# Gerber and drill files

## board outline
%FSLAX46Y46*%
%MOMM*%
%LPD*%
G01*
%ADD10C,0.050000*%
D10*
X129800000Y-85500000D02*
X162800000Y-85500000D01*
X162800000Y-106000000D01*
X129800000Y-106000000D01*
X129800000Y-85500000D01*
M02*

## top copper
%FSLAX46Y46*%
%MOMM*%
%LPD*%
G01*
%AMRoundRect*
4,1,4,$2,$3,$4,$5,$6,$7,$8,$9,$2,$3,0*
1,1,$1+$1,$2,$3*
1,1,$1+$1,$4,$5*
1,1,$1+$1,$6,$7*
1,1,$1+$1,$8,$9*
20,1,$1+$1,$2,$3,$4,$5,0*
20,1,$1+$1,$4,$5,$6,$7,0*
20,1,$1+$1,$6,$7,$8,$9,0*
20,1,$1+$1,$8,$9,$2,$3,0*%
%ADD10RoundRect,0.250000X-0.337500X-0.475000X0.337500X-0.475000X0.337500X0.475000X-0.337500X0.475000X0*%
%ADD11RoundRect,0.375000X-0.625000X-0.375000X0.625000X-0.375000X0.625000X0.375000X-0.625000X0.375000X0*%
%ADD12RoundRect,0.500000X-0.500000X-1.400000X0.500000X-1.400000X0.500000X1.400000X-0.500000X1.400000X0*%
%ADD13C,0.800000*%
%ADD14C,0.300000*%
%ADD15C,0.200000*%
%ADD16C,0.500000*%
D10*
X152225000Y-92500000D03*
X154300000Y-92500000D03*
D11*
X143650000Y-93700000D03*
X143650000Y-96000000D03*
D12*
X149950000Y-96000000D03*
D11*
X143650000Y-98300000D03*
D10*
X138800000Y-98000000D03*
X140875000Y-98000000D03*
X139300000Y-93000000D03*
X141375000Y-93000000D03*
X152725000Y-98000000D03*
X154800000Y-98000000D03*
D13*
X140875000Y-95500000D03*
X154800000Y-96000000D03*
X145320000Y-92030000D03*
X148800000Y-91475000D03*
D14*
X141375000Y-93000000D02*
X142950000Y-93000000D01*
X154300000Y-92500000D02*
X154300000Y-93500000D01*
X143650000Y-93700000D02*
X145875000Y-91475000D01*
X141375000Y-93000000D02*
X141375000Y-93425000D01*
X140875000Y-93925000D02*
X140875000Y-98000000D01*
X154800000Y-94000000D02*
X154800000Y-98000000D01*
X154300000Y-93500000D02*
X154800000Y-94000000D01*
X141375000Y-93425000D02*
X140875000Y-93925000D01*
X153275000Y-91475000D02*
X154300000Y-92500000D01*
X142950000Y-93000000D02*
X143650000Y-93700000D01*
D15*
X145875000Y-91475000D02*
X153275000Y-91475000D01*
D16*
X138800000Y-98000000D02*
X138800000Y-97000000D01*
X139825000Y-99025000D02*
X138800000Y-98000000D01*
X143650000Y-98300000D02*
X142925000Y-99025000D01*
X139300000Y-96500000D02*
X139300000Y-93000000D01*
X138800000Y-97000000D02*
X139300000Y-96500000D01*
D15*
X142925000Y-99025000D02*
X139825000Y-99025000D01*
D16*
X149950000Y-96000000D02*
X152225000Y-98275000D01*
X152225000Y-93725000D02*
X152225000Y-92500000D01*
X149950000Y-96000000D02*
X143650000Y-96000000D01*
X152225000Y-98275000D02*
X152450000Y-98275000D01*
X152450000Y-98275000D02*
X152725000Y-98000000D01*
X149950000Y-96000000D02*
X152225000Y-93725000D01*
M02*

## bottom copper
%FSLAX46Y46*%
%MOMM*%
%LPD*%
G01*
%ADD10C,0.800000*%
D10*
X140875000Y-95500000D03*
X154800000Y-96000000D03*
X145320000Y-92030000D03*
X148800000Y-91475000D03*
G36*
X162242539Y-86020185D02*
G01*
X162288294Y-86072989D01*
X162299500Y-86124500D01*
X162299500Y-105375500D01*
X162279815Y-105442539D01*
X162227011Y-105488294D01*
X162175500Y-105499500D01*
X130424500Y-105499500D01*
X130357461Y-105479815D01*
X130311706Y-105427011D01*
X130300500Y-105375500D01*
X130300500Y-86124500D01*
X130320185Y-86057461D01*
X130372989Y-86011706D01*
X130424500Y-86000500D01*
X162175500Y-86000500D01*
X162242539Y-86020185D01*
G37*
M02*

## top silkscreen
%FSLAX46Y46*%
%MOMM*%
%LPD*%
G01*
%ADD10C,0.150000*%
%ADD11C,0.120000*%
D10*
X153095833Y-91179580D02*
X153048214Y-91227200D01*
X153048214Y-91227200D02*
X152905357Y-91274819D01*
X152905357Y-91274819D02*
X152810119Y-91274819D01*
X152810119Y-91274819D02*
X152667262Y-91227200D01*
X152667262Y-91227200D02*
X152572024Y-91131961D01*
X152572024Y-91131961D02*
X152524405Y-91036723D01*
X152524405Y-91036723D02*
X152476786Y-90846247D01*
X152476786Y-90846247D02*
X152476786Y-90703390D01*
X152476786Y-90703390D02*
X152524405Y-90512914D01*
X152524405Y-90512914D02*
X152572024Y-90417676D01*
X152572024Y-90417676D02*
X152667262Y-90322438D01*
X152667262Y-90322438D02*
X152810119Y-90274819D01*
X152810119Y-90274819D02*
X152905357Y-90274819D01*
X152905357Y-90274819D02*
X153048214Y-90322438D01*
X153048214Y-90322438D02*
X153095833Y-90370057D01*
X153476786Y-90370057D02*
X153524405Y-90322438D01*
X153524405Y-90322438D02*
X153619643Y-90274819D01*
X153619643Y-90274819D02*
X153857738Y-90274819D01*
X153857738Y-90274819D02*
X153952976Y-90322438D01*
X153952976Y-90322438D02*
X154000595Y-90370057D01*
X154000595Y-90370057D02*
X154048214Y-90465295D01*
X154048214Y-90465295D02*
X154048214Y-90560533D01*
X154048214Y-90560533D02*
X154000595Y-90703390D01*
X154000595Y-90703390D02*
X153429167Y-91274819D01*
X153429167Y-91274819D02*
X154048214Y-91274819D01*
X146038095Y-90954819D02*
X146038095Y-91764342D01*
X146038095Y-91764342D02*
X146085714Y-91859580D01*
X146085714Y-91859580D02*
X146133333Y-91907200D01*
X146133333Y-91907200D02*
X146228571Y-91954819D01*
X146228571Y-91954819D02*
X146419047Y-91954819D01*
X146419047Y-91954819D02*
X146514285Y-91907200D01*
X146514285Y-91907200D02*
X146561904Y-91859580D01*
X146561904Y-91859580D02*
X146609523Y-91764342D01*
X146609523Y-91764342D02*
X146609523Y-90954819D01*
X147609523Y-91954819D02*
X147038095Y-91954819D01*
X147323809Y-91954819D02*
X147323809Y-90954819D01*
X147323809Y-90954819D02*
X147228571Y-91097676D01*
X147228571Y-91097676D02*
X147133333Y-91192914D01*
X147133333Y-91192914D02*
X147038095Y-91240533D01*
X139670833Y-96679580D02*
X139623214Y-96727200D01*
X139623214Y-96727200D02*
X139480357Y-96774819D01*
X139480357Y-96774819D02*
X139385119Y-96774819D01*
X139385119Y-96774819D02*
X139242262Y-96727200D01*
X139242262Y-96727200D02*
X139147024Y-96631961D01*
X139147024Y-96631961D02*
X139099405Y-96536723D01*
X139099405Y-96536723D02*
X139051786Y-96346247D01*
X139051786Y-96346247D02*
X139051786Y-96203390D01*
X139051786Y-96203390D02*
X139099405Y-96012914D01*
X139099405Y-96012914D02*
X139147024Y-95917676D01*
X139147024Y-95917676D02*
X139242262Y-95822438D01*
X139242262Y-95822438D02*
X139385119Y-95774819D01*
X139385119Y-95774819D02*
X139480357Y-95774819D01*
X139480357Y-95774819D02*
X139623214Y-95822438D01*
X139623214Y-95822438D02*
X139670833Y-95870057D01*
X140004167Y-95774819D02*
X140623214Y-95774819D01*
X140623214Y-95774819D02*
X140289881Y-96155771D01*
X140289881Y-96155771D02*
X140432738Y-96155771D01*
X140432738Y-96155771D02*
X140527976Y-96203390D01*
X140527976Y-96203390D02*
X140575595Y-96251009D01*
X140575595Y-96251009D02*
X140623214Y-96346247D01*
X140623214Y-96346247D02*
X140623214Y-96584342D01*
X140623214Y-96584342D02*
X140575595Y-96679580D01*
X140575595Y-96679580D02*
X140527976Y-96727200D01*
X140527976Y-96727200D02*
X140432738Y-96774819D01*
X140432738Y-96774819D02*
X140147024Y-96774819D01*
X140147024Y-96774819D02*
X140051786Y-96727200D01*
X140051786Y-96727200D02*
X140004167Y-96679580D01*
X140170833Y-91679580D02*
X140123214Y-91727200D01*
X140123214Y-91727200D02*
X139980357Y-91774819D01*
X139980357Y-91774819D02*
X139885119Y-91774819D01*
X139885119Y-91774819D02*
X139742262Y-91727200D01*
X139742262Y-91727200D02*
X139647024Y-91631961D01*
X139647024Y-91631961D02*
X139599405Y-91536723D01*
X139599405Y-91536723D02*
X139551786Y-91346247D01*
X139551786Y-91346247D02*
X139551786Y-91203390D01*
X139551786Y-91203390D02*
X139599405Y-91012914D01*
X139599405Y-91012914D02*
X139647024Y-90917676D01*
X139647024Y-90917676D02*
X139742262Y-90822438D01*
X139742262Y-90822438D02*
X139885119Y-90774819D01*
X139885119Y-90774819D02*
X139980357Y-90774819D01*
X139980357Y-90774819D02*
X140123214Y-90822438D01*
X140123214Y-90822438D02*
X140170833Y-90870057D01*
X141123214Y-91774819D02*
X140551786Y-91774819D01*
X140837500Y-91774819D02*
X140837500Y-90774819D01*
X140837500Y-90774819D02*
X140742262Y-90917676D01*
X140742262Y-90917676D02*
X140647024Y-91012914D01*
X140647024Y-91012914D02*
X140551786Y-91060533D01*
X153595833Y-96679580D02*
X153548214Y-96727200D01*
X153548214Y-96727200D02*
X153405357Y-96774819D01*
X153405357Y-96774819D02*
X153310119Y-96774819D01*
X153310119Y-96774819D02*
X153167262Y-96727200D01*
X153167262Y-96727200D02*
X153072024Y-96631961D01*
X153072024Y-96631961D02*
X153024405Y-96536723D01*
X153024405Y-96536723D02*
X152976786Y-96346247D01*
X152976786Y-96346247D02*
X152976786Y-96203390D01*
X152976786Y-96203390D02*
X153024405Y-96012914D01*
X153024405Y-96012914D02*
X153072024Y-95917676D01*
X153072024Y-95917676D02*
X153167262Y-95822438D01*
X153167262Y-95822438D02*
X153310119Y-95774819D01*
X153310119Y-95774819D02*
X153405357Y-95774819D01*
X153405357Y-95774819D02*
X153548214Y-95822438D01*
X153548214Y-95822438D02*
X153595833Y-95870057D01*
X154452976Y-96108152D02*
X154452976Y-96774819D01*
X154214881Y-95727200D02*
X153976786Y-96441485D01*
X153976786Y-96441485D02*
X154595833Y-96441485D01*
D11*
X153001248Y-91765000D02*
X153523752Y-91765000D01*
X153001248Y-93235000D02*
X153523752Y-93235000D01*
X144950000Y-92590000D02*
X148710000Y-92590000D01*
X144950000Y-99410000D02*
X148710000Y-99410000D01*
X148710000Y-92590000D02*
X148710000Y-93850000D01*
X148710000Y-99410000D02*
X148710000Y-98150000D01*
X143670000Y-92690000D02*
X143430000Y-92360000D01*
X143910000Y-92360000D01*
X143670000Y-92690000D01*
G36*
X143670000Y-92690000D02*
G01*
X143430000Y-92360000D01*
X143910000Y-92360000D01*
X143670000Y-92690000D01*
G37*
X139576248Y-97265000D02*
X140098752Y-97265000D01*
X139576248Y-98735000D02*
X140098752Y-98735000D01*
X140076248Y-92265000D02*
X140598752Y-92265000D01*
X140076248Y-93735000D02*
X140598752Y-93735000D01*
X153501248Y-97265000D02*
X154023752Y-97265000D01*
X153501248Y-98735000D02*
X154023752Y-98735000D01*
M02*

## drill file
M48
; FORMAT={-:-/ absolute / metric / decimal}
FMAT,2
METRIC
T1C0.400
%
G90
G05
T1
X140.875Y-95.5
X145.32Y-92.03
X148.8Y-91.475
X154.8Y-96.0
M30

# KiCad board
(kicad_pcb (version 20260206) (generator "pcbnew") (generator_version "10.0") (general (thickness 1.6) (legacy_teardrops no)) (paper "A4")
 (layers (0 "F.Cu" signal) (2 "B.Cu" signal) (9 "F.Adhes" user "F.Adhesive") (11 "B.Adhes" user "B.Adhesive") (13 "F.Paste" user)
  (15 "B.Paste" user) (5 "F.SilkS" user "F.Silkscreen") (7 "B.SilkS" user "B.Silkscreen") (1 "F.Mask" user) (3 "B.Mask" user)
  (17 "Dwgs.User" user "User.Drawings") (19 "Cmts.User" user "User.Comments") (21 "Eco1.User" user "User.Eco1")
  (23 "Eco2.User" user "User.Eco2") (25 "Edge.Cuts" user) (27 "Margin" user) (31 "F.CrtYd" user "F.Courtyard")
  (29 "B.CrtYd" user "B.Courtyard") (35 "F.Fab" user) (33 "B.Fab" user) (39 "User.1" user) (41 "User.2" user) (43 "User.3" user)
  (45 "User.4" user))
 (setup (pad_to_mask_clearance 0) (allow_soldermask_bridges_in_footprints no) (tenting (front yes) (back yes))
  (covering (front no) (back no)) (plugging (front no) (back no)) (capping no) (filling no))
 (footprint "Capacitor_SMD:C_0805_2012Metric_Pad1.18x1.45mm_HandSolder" (layer "F.Cu") (at 153.2625 92.5)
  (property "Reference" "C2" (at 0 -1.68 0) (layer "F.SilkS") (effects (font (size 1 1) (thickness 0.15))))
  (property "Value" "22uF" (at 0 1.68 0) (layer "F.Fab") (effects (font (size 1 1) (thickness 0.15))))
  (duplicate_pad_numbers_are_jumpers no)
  (fp_line (start -0.261252 -0.735) (end 0.261252 -0.735) (stroke (width 0.12) (type solid)) (layer "F.SilkS"))
  (fp_line (start -0.261252 0.735) (end 0.261252 0.735) (stroke (width 0.12) (type solid)) (layer "F.SilkS"))
  (pad "1" smd roundrect (at -1.0375 0) (size 1.175 1.45) (layers "F.Cu" "F.Mask" "F.Paste") (roundrect_rratio 0.212766) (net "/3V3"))
  (pad "2" smd roundrect (at 1.0375 0) (size 1.175 1.45) (layers "F.Cu" "F.Mask" "F.Paste") (roundrect_rratio 0.212766) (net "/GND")))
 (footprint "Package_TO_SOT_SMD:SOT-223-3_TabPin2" (layer "F.Cu") (at 146.8 96)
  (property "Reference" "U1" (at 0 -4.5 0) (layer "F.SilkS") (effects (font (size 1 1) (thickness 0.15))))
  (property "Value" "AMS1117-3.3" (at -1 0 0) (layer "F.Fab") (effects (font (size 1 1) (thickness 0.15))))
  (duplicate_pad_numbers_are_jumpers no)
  (fp_line (start -1.85 -3.41) (end 1.91 -3.41) (stroke (width 0.12) (type solid)) (layer "F.SilkS"))
  (fp_line (start -1.85 3.41) (end 1.91 3.41) (stroke (width 0.12) (type solid)) (layer "F.SilkS"))
  (fp_line (start 1.91 -3.41) (end 1.91 -2.15) (stroke (width 0.12) (type solid)) (layer "F.SilkS"))
  (fp_line (start 1.91 3.41) (end 1.91 2.15) (stroke (width 0.12) (type solid)) (layer "F.SilkS"))
  (fp_poly
   (pts (xy -3.13 -3.31) (xy -3.37 -3.64) (xy -2.89 -3.64) (xy -3.13 -3.31)) (stroke (width 0.12) (type solid)) (fill yes) (layer "F.SilkS"))
  (pad "1" smd roundrect (at -3.15 -2.3) (size 2 1.5) (layers "F.Cu" "F.Mask" "F.Paste") (roundrect_rratio 0.25) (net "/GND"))
  (pad "2" smd roundrect (at -3.15 0) (size 2 1.5) (layers "F.Cu" "F.Mask" "F.Paste") (roundrect_rratio 0.25) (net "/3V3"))
  (pad "2" smd roundrect (at 3.15 0) (size 2 3.8) (layers "F.Cu" "F.Mask" "F.Paste") (roundrect_rratio 0.25) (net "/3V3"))
  (pad "3" smd roundrect (at -3.15 2.3) (size 2 1.5) (layers "F.Cu" "F.Mask" "F.Paste") (roundrect_rratio 0.25) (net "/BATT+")))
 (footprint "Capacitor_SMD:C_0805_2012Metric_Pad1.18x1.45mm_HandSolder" (layer "F.Cu") (at 139.8375 98)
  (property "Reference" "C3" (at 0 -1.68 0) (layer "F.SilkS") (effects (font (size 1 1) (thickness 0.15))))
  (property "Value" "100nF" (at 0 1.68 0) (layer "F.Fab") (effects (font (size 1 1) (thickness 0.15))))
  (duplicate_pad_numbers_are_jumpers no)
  (fp_line (start -0.261252 -0.735) (end 0.261252 -0.735) (stroke (width 0.12) (type solid)) (layer "F.SilkS"))
  (fp_line (start -0.261252 0.735) (end 0.261252 0.735) (stroke (width 0.12) (type solid)) (layer "F.SilkS"))
  (pad "1" smd roundrect (at -1.0375 0) (size 1.175 1.45) (layers "F.Cu" "F.Mask" "F.Paste") (roundrect_rratio 0.212766) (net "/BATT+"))
  (pad "2" smd roundrect (at 1.0375 0) (size 1.175 1.45) (layers "F.Cu" "F.Mask" "F.Paste") (roundrect_rratio 0.212766) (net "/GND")))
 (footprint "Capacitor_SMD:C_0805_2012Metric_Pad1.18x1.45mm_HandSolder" (layer "F.Cu") (at 140.3375 93)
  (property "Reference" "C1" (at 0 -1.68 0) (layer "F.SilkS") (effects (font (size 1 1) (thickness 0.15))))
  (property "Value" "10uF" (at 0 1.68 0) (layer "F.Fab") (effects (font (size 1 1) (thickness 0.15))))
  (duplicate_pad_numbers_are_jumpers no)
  (fp_line (start -0.261252 -0.735) (end 0.261252 -0.735) (stroke (width 0.12) (type solid)) (layer "F.SilkS"))
  (fp_line (start -0.261252 0.735) (end 0.261252 0.735) (stroke (width 0.12) (type solid)) (layer "F.SilkS"))
  (pad "1" smd roundrect (at -1.0375 0) (size 1.175 1.45) (layers "F.Cu" "F.Mask" "F.Paste") (roundrect_rratio 0.212766) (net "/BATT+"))
  (pad "2" smd roundrect (at 1.0375 0) (size 1.175 1.45) (layers "F.Cu" "F.Mask" "F.Paste") (roundrect_rratio 0.212766) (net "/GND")))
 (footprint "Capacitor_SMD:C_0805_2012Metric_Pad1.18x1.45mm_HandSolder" (layer "F.Cu") (at 153.7625 98)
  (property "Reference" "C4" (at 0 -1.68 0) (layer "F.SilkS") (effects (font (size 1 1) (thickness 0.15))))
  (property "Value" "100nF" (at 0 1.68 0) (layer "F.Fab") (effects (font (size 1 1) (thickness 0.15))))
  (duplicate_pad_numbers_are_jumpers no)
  (fp_line (start -0.261252 -0.735) (end 0.261252 -0.735) (stroke (width 0.12) (type solid)) (layer "F.SilkS"))
  (fp_line (start -0.261252 0.735) (end 0.261252 0.735) (stroke (width 0.12) (type solid)) (layer "F.SilkS"))
  (pad "1" smd roundrect (at -1.0375 0) (size 1.175 1.45) (layers "F.Cu" "F.Mask" "F.Paste") (roundrect_rratio 0.212766) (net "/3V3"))
  (pad "2" smd roundrect (at 1.0375 0) (size 1.175 1.45) (layers "F.Cu" "F.Mask" "F.Paste") (roundrect_rratio 0.212766) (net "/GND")))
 (gr_rect (start 129.8 85.5) (end 162.8 106) (stroke (width 0.05) (type default)) (fill no) (layer "Edge.Cuts"))
 (segment (start 141.375 93) (end 142.95 93) (width 0.3) (layer "F.Cu") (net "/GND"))
 (segment (start 154.3 92.5) (end 154.3 93.5) (width 0.3) (layer "F.Cu") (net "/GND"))
 (segment (start 143.65 93.7) (end 145.875 91.475) (width 0.3) (layer "F.Cu") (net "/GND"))
 (segment (start 141.375 93) (end 141.375 93.425) (width 0.3) (layer "F.Cu") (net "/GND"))
 (segment (start 140.875 93.925) (end 140.875 98) (width 0.3) (layer "F.Cu") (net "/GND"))
 (segment (start 154.8 94) (end 154.8 98) (width 0.3) (layer "F.Cu") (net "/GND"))
 (segment (start 154.3 93.5) (end 154.8 94) (width 0.3) (layer "F.Cu") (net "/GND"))
 (segment (start 141.375 93.425) (end 140.875 93.925) (width 0.3) (layer "F.Cu") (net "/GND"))
 (segment (start 153.275 91.475) (end 154.3 92.5) (width 0.3) (layer "F.Cu") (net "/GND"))
 (segment (start 142.95 93) (end 143.65 93.7) (width 0.3) (layer "F.Cu") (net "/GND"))
 (segment (start 145.875 91.475) (end 153.275 91.475) (width 0.2) (layer "F.Cu") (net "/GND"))
 (via (at 140.875 95.5) (size 0.8) (drill 0.4) (layers "F.Cu" "B.Cu") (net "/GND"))
 (via (at 154.8 96) (size 0.8) (drill 0.4) (layers "F.Cu" "B.Cu") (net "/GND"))
 (via (at 145.32 92.03) (size 0.8) (drill 0.4) (layers "F.Cu" "B.Cu") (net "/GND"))
 (via (at 148.8 91.475) (size 0.8) (drill 0.4) (layers "F.Cu" "B.Cu") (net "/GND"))
 (segment (start 138.8 98) (end 138.8 97) (width 0.5) (layer "F.Cu") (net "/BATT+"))
 (segment (start 139.825 99.025) (end 138.8 98) (width 0.5) (layer "F.Cu") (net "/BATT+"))
 (segment (start 143.65 98.3) (end 142.925 99.025) (width 0.5) (layer "F.Cu") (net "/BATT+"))
 (segment (start 139.3 96.5) (end 139.3 93) (width 0.5) (layer "F.Cu") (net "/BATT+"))
 (segment (start 138.8 97) (end 139.3 96.5) (width 0.5) (layer "F.Cu") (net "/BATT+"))
 (segment (start 142.925 99.025) (end 139.825 99.025) (width 0.2) (layer "F.Cu") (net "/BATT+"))
 (segment (start 149.95 96) (end 152.225 98.275) (width 0.5) (layer "F.Cu") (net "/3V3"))
 (segment (start 152.225 93.725) (end 152.225 92.5) (width 0.5) (layer "F.Cu") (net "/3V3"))
 (segment (start 149.95 96) (end 143.65 96) (width 0.5) (layer "F.Cu") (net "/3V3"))
 (segment (start 152.225 98.275) (end 152.45 98.275) (width 0.5) (layer "F.Cu") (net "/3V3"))
 (segment (start 152.45 98.275) (end 152.725 98) (width 0.5) (layer "F.Cu") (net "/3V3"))
 (segment (start 149.95 96) (end 152.225 93.725) (width 0.5) (layer "F.Cu") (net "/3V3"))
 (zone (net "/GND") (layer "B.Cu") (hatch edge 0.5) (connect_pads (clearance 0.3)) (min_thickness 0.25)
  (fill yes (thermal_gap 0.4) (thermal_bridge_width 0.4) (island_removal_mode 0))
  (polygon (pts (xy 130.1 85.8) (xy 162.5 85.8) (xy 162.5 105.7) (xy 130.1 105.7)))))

